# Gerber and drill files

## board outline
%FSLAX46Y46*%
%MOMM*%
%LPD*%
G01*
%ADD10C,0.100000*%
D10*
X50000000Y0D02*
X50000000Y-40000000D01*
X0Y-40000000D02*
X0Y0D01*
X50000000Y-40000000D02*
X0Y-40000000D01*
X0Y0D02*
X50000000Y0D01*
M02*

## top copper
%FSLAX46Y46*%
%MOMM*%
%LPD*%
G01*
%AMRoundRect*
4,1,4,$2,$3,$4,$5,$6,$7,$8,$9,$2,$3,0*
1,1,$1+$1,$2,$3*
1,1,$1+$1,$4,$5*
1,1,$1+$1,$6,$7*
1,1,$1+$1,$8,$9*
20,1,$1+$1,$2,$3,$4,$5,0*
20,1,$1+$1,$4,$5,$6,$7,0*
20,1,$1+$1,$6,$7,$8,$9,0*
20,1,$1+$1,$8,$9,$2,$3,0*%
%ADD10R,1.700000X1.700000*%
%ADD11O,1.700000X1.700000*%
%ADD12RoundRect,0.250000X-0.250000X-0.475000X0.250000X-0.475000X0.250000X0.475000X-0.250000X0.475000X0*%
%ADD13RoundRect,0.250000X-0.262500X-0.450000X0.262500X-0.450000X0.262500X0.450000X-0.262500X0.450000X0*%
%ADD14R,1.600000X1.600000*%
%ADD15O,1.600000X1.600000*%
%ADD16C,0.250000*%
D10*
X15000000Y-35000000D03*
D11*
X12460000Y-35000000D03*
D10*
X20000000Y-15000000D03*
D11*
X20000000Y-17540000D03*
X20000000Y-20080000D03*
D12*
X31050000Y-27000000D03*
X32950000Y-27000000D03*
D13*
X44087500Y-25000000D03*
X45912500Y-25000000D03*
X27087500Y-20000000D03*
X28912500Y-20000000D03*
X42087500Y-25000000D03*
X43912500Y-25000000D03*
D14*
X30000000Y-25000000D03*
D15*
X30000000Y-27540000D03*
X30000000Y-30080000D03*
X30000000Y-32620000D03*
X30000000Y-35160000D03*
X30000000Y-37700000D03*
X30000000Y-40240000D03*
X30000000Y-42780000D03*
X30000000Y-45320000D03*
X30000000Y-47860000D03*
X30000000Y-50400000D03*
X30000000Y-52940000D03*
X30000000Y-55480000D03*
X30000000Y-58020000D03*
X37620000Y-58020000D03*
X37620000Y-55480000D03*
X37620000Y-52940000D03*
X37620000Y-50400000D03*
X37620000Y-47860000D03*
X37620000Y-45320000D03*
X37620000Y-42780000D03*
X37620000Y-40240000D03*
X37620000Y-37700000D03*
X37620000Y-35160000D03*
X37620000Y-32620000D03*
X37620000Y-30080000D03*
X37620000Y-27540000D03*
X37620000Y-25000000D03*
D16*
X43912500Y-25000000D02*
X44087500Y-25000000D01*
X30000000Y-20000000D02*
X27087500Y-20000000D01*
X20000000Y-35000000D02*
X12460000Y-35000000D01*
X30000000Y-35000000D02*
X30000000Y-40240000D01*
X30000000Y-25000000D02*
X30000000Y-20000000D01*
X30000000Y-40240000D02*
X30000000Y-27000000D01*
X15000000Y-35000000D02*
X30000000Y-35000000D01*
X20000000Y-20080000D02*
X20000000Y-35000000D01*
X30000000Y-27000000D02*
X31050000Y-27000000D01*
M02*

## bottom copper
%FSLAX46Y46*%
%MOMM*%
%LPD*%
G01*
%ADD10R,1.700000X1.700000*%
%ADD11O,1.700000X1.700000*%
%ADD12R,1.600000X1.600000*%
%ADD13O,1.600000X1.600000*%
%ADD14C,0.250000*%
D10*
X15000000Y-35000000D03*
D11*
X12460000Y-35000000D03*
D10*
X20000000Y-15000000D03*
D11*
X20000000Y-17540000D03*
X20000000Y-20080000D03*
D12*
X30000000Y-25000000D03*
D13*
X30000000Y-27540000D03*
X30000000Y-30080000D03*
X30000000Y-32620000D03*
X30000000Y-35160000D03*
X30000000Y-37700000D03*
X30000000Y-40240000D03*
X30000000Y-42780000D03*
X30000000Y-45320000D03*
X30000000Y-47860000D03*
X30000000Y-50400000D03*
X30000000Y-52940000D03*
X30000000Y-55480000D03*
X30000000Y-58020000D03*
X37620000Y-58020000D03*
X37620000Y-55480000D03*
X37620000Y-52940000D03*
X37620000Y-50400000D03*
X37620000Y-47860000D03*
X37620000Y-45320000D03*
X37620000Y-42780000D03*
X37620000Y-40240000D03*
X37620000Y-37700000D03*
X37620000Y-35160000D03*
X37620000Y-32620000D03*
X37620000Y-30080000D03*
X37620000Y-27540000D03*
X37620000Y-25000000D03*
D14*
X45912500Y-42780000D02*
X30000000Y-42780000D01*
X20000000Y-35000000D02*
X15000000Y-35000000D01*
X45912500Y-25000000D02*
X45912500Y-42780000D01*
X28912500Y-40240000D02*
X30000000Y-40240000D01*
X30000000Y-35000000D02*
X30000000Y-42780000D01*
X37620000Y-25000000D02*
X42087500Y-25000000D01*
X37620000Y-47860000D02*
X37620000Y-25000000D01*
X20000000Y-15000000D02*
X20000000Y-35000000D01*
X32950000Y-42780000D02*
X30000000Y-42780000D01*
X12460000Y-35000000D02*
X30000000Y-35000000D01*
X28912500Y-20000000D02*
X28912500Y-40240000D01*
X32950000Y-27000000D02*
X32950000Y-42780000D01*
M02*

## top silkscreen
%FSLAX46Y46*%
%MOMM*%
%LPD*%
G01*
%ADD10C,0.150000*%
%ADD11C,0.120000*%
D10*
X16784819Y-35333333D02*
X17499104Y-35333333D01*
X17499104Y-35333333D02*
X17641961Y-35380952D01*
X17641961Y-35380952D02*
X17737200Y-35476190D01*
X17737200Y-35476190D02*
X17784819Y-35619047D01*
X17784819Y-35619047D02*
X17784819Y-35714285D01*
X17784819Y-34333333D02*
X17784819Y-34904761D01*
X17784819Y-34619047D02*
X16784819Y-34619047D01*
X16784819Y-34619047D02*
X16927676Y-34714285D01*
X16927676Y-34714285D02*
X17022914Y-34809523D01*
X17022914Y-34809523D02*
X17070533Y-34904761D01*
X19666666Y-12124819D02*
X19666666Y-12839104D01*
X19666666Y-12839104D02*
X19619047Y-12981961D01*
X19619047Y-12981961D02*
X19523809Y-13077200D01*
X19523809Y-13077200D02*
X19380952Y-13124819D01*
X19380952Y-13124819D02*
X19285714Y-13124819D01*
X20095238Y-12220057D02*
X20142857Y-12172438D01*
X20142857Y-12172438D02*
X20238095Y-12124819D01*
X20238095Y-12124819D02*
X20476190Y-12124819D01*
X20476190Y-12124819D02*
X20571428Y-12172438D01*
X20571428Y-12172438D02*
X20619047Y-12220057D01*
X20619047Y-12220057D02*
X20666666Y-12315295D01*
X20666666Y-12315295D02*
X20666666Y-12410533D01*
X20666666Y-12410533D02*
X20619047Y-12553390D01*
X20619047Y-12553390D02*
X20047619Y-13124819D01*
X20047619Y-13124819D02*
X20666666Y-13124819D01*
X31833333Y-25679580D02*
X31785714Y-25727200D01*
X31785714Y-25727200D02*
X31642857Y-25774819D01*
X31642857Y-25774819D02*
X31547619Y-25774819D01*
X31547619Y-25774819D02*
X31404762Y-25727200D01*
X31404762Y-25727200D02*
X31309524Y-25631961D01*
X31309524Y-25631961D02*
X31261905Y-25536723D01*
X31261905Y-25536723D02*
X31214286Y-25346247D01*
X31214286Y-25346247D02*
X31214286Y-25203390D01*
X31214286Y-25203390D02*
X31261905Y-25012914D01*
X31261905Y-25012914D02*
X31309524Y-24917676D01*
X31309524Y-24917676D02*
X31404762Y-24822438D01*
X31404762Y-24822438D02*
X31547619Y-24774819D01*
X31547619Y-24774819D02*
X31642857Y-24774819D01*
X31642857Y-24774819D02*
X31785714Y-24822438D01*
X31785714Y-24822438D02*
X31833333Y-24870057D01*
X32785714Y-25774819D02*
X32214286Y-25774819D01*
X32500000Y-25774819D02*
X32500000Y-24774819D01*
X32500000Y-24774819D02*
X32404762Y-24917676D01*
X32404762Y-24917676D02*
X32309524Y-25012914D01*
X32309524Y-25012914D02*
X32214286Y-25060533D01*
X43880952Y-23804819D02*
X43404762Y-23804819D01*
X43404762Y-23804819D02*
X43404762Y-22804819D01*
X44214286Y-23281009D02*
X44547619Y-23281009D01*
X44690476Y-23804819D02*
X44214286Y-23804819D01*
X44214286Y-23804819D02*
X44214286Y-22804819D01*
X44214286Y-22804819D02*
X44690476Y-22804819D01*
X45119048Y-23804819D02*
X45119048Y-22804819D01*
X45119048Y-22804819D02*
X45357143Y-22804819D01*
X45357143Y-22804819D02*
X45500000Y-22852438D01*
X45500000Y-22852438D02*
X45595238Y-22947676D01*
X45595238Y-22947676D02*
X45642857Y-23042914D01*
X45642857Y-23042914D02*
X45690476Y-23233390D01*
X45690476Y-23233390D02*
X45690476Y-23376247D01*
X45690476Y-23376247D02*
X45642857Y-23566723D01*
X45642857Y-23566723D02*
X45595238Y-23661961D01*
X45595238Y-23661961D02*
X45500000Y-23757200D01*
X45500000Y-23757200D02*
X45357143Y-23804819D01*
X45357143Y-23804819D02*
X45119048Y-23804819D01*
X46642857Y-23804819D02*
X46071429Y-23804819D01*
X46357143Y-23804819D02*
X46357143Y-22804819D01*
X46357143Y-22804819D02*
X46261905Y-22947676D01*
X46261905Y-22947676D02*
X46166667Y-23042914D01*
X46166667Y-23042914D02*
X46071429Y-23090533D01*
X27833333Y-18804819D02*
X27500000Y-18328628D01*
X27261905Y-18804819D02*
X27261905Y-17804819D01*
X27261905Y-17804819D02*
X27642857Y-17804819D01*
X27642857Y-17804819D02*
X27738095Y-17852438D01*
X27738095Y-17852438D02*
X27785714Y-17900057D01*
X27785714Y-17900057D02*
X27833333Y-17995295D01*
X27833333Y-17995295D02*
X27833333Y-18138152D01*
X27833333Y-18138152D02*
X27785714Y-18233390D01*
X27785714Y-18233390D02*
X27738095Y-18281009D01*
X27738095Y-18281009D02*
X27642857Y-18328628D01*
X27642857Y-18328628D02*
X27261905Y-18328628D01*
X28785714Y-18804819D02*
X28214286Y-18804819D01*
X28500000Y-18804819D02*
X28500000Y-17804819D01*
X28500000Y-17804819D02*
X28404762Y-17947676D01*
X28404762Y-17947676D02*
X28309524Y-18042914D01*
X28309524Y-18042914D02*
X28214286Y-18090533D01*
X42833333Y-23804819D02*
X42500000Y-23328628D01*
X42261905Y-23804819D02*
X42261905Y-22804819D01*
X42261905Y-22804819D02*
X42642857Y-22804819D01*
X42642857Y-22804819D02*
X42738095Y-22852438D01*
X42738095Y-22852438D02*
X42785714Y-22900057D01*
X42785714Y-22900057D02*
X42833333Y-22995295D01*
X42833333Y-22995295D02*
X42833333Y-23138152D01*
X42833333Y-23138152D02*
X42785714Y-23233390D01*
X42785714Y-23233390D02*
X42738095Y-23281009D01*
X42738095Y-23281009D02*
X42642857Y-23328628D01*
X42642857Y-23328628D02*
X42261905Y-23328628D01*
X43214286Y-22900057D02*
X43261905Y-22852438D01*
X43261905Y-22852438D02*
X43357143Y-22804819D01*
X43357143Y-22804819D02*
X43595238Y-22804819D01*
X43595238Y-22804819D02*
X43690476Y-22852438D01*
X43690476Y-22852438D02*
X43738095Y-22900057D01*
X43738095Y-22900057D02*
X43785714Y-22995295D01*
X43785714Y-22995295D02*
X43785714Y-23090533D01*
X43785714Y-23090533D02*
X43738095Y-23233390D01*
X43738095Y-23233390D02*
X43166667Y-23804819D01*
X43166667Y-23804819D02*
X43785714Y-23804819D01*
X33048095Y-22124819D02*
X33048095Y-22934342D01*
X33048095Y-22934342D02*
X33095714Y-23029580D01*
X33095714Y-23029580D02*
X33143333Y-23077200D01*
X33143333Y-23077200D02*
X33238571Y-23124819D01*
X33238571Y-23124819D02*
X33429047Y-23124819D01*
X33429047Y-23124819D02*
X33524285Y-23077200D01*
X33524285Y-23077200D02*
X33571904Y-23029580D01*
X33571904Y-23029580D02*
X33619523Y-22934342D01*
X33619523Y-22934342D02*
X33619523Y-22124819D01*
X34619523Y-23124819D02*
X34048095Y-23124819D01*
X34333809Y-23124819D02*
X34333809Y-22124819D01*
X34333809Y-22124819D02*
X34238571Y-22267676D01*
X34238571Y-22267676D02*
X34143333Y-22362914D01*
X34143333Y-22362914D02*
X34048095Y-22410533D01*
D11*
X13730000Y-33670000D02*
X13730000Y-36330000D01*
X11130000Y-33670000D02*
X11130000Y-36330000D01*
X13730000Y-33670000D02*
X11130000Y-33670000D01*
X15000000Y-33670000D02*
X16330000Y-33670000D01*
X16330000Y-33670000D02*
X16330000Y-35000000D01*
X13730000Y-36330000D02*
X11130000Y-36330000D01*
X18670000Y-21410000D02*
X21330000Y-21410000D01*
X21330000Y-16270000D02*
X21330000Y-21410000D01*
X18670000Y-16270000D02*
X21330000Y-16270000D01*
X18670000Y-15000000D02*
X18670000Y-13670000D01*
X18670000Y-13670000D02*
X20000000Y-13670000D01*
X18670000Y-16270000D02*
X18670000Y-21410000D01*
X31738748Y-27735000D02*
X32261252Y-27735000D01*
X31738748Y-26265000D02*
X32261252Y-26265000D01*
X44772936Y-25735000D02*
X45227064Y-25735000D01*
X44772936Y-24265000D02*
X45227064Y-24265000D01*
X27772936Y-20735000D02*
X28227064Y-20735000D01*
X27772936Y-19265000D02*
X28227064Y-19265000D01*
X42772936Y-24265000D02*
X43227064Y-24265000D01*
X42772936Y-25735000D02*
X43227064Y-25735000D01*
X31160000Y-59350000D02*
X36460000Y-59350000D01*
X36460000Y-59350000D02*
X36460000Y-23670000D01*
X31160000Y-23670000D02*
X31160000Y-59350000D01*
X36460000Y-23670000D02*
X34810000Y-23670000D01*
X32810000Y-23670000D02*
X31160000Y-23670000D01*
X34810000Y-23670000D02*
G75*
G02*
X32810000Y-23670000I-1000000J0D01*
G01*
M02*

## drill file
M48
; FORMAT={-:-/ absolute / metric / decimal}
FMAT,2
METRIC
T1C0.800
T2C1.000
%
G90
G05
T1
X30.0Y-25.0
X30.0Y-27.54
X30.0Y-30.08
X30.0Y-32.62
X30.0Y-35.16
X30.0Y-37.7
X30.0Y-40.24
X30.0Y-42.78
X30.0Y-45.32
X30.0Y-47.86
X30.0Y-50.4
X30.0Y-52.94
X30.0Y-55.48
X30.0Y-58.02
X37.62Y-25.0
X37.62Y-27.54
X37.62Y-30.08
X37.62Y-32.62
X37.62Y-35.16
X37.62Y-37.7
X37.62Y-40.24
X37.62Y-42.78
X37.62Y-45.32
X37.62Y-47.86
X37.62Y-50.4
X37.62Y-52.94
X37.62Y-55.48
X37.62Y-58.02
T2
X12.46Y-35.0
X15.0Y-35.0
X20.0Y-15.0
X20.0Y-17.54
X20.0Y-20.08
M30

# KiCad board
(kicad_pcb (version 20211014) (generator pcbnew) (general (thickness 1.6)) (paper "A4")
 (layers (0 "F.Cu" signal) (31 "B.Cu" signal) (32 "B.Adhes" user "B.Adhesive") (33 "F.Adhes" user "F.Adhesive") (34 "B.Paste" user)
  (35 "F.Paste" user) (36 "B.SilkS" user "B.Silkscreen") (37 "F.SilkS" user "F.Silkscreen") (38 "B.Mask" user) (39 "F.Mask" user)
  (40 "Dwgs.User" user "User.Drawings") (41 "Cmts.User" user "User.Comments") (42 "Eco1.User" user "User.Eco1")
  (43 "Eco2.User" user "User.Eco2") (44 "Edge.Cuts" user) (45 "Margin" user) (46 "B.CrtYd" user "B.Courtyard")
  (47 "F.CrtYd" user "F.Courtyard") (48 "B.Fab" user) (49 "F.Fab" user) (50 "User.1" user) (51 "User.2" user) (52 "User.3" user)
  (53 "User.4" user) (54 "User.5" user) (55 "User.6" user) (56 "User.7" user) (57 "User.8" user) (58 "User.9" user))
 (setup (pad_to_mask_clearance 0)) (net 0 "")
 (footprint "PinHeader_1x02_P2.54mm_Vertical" (layer "F.Cu") (at 15 35 -90)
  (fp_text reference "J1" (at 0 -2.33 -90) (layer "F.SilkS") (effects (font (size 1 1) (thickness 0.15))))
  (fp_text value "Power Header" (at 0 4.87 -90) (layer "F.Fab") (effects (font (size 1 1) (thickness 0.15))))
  (fp_line (start -1.33 1.27) (end 1.33 1.27) (layer "F.SilkS") (width 0.12))
  (fp_line (start -1.33 3.87) (end 1.33 3.87) (layer "F.SilkS") (width 0.12))
  (fp_line (start -1.33 1.27) (end -1.33 3.87) (layer "F.SilkS") (width 0.12))
  (fp_line (start -1.33 0) (end -1.33 -1.33) (layer "F.SilkS") (width 0.12))
  (fp_line (start -1.33 -1.33) (end 0 -1.33) (layer "F.SilkS") (width 0.12))
  (fp_line (start 1.33 1.27) (end 1.33 3.87) (layer "F.SilkS") (width 0.12))
  (pad "1" thru_hole rect (at 0 0 270) (size 1.7 1.7) (drill 1) (layers *.Cu *.Mask))
  (pad "2" thru_hole oval (at 0 2.54 270) (size 1.7 1.7) (drill 1) (layers *.Cu *.Mask)))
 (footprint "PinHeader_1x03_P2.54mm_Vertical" (layer "F.Cu") (at 20 15)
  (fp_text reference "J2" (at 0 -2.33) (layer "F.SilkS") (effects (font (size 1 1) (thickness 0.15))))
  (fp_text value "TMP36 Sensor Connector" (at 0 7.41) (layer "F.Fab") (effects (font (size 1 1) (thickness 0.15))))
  (fp_line (start -1.33 6.41) (end 1.33 6.41) (layer "F.SilkS") (width 0.12))
  (fp_line (start 1.33 1.27) (end 1.33 6.41) (layer "F.SilkS") (width 0.12))
  (fp_line (start -1.33 1.27) (end 1.33 1.27) (layer "F.SilkS") (width 0.12))
  (fp_line (start -1.33 0) (end -1.33 -1.33) (layer "F.SilkS") (width 0.12))
  (fp_line (start -1.33 -1.33) (end 0 -1.33) (layer "F.SilkS") (width 0.12))
  (fp_line (start -1.33 1.27) (end -1.33 6.41) (layer "F.SilkS") (width 0.12))
  (pad "1" thru_hole rect (at 0 0) (size 1.7 1.7) (drill 1) (layers *.Cu *.Mask))
  (pad "2" thru_hole oval (at 0 2.54) (size 1.7 1.7) (drill 1) (layers *.Cu *.Mask))
  (pad "3" thru_hole oval (at 0 5.08) (size 1.7 1.7) (drill 1) (layers *.Cu *.Mask)))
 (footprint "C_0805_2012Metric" (layer "F.Cu") (at 32 27)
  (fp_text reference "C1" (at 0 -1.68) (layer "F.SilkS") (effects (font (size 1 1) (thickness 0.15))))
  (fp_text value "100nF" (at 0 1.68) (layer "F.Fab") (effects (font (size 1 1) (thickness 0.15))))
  (fp_line (start -0.261252 0.735) (end 0.261252 0.735) (layer "F.SilkS") (width 0.12))
  (fp_line (start -0.261252 -0.735) (end 0.261252 -0.735) (layer "F.SilkS") (width 0.12))
  (pad "1" smd roundrect (at -0.95 0) (size 1 1.45) (layers "F.Cu" "F.Paste" "F.Mask") (roundrect_rratio 0.25))
  (pad "2" smd roundrect (at 0.95 0) (size 1 1.45) (layers "F.Cu" "F.Paste" "F.Mask") (roundrect_rratio 0.25)))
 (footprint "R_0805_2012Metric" (layer "F.Cu") (at 45 25)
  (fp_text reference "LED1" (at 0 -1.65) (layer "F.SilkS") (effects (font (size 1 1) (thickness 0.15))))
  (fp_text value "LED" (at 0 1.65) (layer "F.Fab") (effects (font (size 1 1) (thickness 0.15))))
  (fp_line (start -0.227064 0.735) (end 0.227064 0.735) (layer "F.SilkS") (width 0.12))
  (fp_line (start -0.227064 -0.735) (end 0.227064 -0.735) (layer "F.SilkS") (width 0.12))
  (pad "1" smd roundrect (at -0.9125 0) (size 1.025 1.4) (layers "F.Cu" "F.Paste" "F.Mask") (roundrect_rratio 0.243902))
  (pad "2" smd roundrect (at 0.9125 0) (size 1.025 1.4) (layers "F.Cu" "F.Paste" "F.Mask") (roundrect_rratio 0.243902)))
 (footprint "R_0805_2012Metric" (layer "F.Cu") (at 28 20)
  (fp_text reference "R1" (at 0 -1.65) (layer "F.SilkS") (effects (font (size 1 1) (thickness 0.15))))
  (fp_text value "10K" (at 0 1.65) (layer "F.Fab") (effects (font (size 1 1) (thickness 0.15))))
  (fp_line (start -0.227064 0.735) (end 0.227064 0.735) (layer "F.SilkS") (width 0.12))
  (fp_line (start -0.227064 -0.735) (end 0.227064 -0.735) (layer "F.SilkS") (width 0.12))
  (pad "1" smd roundrect (at -0.9125 0) (size 1.025 1.4) (layers "F.Cu" "F.Paste" "F.Mask") (roundrect_rratio 0.243902))
  (pad "2" smd roundrect (at 0.9125 0) (size 1.025 1.4) (layers "F.Cu" "F.Paste" "F.Mask") (roundrect_rratio 0.243902)))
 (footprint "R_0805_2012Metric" (layer "F.Cu") (at 43 25)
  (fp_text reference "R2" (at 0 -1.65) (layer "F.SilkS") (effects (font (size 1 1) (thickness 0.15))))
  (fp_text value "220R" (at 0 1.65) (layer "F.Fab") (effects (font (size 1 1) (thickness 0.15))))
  (fp_line (start -0.227064 -0.735) (end 0.227064 -0.735) (layer "F.SilkS") (width 0.12))
  (fp_line (start -0.227064 0.735) (end 0.227064 0.735) (layer "F.SilkS") (width 0.12))
  (pad "1" smd roundrect (at -0.9125 0) (size 1.025 1.4) (layers "F.Cu" "F.Paste" "F.Mask") (roundrect_rratio 0.243902))
  (pad "2" smd roundrect (at 0.9125 0) (size 1.025 1.4) (layers "F.Cu" "F.Paste" "F.Mask") (roundrect_rratio 0.243902)))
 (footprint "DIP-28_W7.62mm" (layer "F.Cu") (at 30 25)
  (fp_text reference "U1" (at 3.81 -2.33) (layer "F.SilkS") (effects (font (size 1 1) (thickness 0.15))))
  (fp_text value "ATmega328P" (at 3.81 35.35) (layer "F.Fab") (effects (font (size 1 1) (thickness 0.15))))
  (fp_line (start 1.16 34.35) (end 6.46 34.35) (layer "F.SilkS") (width 0.12))
  (fp_line (start 6.46 34.35) (end 6.46 -1.33) (layer "F.SilkS") (width 0.12))
  (fp_line (start 1.16 -1.33) (end 1.16 34.35) (layer "F.SilkS") (width 0.12))
  (fp_line (start 6.46 -1.33) (end 4.81 -1.33) (layer "F.SilkS") (width 0.12))
  (fp_line (start 2.81 -1.33) (end 1.16 -1.33) (layer "F.SilkS") (width 0.12))
  (fp_arc (start 4.81 -1.33) (mid 3.81 -0.33) (end 2.81 -1.33) (layer "F.SilkS") (width 0.12))
  (pad "1" thru_hole rect (at 0 0) (size 1.6 1.6) (drill 0.8) (layers *.Cu *.Mask))
  (pad "2" thru_hole oval (at 0 2.54) (size 1.6 1.6) (drill 0.8) (layers *.Cu *.Mask))
  (pad "3" thru_hole oval (at 0 5.08) (size 1.6 1.6) (drill 0.8) (layers *.Cu *.Mask))
  (pad "4" thru_hole oval (at 0 7.62) (size 1.6 1.6) (drill 0.8) (layers *.Cu *.Mask))
  (pad "5" thru_hole oval (at 0 10.16) (size 1.6 1.6) (drill 0.8) (layers *.Cu *.Mask))
  (pad "6" thru_hole oval (at 0 12.7) (size 1.6 1.6) (drill 0.8) (layers *.Cu *.Mask))
  (pad "7" thru_hole oval (at 0 15.24) (size 1.6 1.6) (drill 0.8) (layers *.Cu *.Mask))
  (pad "8" thru_hole oval (at 0 17.78) (size 1.6 1.6) (drill 0.8) (layers *.Cu *.Mask))
  (pad "9" thru_hole oval (at 0 20.32) (size 1.6 1.6) (drill 0.8) (layers *.Cu *.Mask))
  (pad "10" thru_hole oval (at 0 22.86) (size 1.6 1.6) (drill 0.8) (layers *.Cu *.Mask))
  (pad "11" thru_hole oval (at 0 25.4) (size 1.6 1.6) (drill 0.8) (layers *.Cu *.Mask))
  (pad "12" thru_hole oval (at 0 27.94) (size 1.6 1.6) (drill 0.8) (layers *.Cu *.Mask))
  (pad "13" thru_hole oval (at 0 30.48) (size 1.6 1.6) (drill 0.8) (layers *.Cu *.Mask))
  (pad "14" thru_hole oval (at 0 33.02) (size 1.6 1.6) (drill 0.8) (layers *.Cu *.Mask))
  (pad "15" thru_hole oval (at 7.62 33.02) (size 1.6 1.6) (drill 0.8) (layers *.Cu *.Mask))
  (pad "16" thru_hole oval (at 7.62 30.48) (size 1.6 1.6) (drill 0.8) (layers *.Cu *.Mask))
  (pad "17" thru_hole oval (at 7.62 27.94) (size 1.6 1.6) (drill 0.8) (layers *.Cu *.Mask))
  (pad "18" thru_hole oval (at 7.62 25.4) (size 1.6 1.6) (drill 0.8) (layers *.Cu *.Mask))
  (pad "19" thru_hole oval (at 7.62 22.86) (size 1.6 1.6) (drill 0.8) (layers *.Cu *.Mask))
  (pad "20" thru_hole oval (at 7.62 20.32) (size 1.6 1.6) (drill 0.8) (layers *.Cu *.Mask))
  (pad "21" thru_hole oval (at 7.62 17.78) (size 1.6 1.6) (drill 0.8) (layers *.Cu *.Mask))
  (pad "22" thru_hole oval (at 7.62 15.24) (size 1.6 1.6) (drill 0.8) (layers *.Cu *.Mask))
  (pad "23" thru_hole oval (at 7.62 12.7) (size 1.6 1.6) (drill 0.8) (layers *.Cu *.Mask))
  (pad "24" thru_hole oval (at 7.62 10.16) (size 1.6 1.6) (drill 0.8) (layers *.Cu *.Mask))
  (pad "25" thru_hole oval (at 7.62 7.62) (size 1.6 1.6) (drill 0.8) (layers *.Cu *.Mask))
  (pad "26" thru_hole oval (at 7.62 5.08) (size 1.6 1.6) (drill 0.8) (layers *.Cu *.Mask))
  (pad "27" thru_hole oval (at 7.62 2.54) (size 1.6 1.6) (drill 0.8) (layers *.Cu *.Mask))
  (pad "28" thru_hole oval (at 7.62 0) (size 1.6 1.6) (drill 0.8) (layers *.Cu *.Mask)))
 (gr_line (start 50 0) (end 50 40) (layer "Edge.Cuts") (width 0.1))
 (gr_line (start 0 40) (end 0 0) (layer "Edge.Cuts") (width 0.1))
 (gr_line (start 50 40) (end 0 40) (layer "Edge.Cuts") (width 0.1))
 (gr_line (start 0 0) (end 50 0) (layer "Edge.Cuts") (width 0.1))
 (segment (start 43.9125 25) (end 44.0875 25) (width 0.25) (layer "F.Cu") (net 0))
 (segment (start 30 20) (end 27.0875 20) (width 0.25) (layer "F.Cu") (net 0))
 (segment (start 20 35) (end 12.46 35) (width 0.25) (layer "F.Cu") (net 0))
 (segment (start 30 35) (end 30 40.24) (width 0.25) (layer "F.Cu") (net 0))
 (segment (start 30 25) (end 30 20) (width 0.25) (layer "F.Cu") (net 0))
 (segment (start 30 40.24) (end 30 27) (width 0.25) (layer "F.Cu") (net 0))
 (segment (start 15 35) (end 30 35) (width 0.25) (layer "F.Cu") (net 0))
 (segment (start 20 20.08) (end 20 35) (width 0.25) (layer "F.Cu") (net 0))
 (segment (start 30 27) (end 31.05 27) (width 0.25) (layer "F.Cu") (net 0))
 (segment (start 45.9125 42.78) (end 30 42.78) (width 0.25) (layer "B.Cu") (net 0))
 (segment (start 20 35) (end 15 35) (width 0.25) (layer "B.Cu") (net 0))
 (segment (start 45.9125 25) (end 45.9125 42.78) (width 0.25) (layer "B.Cu") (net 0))
 (segment (start 28.9125 40.24) (end 30 40.24) (width 0.25) (layer "B.Cu") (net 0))
 (segment (start 30 35) (end 30 42.78) (width 0.25) (layer "B.Cu") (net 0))
 (segment (start 37.62 25) (end 42.0875 25) (width 0.25) (layer "B.Cu") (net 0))
 (segment (start 37.62 47.86) (end 37.62 25) (width 0.25) (layer "B.Cu") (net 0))
 (segment (start 20 15) (end 20 35) (width 0.25) (layer "B.Cu") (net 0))
 (segment (start 32.95 42.78) (end 30 42.78) (width 0.25) (layer "B.Cu") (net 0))
 (segment (start 12.46 35) (end 30 35) (width 0.25) (layer "B.Cu") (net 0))
 (segment (start 28.9125 20) (end 28.9125 40.24) (width 0.25) (layer "B.Cu") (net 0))
 (segment (start 32.95 27) (end 32.95 42.78) (width 0.25) (layer "B.Cu") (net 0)))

